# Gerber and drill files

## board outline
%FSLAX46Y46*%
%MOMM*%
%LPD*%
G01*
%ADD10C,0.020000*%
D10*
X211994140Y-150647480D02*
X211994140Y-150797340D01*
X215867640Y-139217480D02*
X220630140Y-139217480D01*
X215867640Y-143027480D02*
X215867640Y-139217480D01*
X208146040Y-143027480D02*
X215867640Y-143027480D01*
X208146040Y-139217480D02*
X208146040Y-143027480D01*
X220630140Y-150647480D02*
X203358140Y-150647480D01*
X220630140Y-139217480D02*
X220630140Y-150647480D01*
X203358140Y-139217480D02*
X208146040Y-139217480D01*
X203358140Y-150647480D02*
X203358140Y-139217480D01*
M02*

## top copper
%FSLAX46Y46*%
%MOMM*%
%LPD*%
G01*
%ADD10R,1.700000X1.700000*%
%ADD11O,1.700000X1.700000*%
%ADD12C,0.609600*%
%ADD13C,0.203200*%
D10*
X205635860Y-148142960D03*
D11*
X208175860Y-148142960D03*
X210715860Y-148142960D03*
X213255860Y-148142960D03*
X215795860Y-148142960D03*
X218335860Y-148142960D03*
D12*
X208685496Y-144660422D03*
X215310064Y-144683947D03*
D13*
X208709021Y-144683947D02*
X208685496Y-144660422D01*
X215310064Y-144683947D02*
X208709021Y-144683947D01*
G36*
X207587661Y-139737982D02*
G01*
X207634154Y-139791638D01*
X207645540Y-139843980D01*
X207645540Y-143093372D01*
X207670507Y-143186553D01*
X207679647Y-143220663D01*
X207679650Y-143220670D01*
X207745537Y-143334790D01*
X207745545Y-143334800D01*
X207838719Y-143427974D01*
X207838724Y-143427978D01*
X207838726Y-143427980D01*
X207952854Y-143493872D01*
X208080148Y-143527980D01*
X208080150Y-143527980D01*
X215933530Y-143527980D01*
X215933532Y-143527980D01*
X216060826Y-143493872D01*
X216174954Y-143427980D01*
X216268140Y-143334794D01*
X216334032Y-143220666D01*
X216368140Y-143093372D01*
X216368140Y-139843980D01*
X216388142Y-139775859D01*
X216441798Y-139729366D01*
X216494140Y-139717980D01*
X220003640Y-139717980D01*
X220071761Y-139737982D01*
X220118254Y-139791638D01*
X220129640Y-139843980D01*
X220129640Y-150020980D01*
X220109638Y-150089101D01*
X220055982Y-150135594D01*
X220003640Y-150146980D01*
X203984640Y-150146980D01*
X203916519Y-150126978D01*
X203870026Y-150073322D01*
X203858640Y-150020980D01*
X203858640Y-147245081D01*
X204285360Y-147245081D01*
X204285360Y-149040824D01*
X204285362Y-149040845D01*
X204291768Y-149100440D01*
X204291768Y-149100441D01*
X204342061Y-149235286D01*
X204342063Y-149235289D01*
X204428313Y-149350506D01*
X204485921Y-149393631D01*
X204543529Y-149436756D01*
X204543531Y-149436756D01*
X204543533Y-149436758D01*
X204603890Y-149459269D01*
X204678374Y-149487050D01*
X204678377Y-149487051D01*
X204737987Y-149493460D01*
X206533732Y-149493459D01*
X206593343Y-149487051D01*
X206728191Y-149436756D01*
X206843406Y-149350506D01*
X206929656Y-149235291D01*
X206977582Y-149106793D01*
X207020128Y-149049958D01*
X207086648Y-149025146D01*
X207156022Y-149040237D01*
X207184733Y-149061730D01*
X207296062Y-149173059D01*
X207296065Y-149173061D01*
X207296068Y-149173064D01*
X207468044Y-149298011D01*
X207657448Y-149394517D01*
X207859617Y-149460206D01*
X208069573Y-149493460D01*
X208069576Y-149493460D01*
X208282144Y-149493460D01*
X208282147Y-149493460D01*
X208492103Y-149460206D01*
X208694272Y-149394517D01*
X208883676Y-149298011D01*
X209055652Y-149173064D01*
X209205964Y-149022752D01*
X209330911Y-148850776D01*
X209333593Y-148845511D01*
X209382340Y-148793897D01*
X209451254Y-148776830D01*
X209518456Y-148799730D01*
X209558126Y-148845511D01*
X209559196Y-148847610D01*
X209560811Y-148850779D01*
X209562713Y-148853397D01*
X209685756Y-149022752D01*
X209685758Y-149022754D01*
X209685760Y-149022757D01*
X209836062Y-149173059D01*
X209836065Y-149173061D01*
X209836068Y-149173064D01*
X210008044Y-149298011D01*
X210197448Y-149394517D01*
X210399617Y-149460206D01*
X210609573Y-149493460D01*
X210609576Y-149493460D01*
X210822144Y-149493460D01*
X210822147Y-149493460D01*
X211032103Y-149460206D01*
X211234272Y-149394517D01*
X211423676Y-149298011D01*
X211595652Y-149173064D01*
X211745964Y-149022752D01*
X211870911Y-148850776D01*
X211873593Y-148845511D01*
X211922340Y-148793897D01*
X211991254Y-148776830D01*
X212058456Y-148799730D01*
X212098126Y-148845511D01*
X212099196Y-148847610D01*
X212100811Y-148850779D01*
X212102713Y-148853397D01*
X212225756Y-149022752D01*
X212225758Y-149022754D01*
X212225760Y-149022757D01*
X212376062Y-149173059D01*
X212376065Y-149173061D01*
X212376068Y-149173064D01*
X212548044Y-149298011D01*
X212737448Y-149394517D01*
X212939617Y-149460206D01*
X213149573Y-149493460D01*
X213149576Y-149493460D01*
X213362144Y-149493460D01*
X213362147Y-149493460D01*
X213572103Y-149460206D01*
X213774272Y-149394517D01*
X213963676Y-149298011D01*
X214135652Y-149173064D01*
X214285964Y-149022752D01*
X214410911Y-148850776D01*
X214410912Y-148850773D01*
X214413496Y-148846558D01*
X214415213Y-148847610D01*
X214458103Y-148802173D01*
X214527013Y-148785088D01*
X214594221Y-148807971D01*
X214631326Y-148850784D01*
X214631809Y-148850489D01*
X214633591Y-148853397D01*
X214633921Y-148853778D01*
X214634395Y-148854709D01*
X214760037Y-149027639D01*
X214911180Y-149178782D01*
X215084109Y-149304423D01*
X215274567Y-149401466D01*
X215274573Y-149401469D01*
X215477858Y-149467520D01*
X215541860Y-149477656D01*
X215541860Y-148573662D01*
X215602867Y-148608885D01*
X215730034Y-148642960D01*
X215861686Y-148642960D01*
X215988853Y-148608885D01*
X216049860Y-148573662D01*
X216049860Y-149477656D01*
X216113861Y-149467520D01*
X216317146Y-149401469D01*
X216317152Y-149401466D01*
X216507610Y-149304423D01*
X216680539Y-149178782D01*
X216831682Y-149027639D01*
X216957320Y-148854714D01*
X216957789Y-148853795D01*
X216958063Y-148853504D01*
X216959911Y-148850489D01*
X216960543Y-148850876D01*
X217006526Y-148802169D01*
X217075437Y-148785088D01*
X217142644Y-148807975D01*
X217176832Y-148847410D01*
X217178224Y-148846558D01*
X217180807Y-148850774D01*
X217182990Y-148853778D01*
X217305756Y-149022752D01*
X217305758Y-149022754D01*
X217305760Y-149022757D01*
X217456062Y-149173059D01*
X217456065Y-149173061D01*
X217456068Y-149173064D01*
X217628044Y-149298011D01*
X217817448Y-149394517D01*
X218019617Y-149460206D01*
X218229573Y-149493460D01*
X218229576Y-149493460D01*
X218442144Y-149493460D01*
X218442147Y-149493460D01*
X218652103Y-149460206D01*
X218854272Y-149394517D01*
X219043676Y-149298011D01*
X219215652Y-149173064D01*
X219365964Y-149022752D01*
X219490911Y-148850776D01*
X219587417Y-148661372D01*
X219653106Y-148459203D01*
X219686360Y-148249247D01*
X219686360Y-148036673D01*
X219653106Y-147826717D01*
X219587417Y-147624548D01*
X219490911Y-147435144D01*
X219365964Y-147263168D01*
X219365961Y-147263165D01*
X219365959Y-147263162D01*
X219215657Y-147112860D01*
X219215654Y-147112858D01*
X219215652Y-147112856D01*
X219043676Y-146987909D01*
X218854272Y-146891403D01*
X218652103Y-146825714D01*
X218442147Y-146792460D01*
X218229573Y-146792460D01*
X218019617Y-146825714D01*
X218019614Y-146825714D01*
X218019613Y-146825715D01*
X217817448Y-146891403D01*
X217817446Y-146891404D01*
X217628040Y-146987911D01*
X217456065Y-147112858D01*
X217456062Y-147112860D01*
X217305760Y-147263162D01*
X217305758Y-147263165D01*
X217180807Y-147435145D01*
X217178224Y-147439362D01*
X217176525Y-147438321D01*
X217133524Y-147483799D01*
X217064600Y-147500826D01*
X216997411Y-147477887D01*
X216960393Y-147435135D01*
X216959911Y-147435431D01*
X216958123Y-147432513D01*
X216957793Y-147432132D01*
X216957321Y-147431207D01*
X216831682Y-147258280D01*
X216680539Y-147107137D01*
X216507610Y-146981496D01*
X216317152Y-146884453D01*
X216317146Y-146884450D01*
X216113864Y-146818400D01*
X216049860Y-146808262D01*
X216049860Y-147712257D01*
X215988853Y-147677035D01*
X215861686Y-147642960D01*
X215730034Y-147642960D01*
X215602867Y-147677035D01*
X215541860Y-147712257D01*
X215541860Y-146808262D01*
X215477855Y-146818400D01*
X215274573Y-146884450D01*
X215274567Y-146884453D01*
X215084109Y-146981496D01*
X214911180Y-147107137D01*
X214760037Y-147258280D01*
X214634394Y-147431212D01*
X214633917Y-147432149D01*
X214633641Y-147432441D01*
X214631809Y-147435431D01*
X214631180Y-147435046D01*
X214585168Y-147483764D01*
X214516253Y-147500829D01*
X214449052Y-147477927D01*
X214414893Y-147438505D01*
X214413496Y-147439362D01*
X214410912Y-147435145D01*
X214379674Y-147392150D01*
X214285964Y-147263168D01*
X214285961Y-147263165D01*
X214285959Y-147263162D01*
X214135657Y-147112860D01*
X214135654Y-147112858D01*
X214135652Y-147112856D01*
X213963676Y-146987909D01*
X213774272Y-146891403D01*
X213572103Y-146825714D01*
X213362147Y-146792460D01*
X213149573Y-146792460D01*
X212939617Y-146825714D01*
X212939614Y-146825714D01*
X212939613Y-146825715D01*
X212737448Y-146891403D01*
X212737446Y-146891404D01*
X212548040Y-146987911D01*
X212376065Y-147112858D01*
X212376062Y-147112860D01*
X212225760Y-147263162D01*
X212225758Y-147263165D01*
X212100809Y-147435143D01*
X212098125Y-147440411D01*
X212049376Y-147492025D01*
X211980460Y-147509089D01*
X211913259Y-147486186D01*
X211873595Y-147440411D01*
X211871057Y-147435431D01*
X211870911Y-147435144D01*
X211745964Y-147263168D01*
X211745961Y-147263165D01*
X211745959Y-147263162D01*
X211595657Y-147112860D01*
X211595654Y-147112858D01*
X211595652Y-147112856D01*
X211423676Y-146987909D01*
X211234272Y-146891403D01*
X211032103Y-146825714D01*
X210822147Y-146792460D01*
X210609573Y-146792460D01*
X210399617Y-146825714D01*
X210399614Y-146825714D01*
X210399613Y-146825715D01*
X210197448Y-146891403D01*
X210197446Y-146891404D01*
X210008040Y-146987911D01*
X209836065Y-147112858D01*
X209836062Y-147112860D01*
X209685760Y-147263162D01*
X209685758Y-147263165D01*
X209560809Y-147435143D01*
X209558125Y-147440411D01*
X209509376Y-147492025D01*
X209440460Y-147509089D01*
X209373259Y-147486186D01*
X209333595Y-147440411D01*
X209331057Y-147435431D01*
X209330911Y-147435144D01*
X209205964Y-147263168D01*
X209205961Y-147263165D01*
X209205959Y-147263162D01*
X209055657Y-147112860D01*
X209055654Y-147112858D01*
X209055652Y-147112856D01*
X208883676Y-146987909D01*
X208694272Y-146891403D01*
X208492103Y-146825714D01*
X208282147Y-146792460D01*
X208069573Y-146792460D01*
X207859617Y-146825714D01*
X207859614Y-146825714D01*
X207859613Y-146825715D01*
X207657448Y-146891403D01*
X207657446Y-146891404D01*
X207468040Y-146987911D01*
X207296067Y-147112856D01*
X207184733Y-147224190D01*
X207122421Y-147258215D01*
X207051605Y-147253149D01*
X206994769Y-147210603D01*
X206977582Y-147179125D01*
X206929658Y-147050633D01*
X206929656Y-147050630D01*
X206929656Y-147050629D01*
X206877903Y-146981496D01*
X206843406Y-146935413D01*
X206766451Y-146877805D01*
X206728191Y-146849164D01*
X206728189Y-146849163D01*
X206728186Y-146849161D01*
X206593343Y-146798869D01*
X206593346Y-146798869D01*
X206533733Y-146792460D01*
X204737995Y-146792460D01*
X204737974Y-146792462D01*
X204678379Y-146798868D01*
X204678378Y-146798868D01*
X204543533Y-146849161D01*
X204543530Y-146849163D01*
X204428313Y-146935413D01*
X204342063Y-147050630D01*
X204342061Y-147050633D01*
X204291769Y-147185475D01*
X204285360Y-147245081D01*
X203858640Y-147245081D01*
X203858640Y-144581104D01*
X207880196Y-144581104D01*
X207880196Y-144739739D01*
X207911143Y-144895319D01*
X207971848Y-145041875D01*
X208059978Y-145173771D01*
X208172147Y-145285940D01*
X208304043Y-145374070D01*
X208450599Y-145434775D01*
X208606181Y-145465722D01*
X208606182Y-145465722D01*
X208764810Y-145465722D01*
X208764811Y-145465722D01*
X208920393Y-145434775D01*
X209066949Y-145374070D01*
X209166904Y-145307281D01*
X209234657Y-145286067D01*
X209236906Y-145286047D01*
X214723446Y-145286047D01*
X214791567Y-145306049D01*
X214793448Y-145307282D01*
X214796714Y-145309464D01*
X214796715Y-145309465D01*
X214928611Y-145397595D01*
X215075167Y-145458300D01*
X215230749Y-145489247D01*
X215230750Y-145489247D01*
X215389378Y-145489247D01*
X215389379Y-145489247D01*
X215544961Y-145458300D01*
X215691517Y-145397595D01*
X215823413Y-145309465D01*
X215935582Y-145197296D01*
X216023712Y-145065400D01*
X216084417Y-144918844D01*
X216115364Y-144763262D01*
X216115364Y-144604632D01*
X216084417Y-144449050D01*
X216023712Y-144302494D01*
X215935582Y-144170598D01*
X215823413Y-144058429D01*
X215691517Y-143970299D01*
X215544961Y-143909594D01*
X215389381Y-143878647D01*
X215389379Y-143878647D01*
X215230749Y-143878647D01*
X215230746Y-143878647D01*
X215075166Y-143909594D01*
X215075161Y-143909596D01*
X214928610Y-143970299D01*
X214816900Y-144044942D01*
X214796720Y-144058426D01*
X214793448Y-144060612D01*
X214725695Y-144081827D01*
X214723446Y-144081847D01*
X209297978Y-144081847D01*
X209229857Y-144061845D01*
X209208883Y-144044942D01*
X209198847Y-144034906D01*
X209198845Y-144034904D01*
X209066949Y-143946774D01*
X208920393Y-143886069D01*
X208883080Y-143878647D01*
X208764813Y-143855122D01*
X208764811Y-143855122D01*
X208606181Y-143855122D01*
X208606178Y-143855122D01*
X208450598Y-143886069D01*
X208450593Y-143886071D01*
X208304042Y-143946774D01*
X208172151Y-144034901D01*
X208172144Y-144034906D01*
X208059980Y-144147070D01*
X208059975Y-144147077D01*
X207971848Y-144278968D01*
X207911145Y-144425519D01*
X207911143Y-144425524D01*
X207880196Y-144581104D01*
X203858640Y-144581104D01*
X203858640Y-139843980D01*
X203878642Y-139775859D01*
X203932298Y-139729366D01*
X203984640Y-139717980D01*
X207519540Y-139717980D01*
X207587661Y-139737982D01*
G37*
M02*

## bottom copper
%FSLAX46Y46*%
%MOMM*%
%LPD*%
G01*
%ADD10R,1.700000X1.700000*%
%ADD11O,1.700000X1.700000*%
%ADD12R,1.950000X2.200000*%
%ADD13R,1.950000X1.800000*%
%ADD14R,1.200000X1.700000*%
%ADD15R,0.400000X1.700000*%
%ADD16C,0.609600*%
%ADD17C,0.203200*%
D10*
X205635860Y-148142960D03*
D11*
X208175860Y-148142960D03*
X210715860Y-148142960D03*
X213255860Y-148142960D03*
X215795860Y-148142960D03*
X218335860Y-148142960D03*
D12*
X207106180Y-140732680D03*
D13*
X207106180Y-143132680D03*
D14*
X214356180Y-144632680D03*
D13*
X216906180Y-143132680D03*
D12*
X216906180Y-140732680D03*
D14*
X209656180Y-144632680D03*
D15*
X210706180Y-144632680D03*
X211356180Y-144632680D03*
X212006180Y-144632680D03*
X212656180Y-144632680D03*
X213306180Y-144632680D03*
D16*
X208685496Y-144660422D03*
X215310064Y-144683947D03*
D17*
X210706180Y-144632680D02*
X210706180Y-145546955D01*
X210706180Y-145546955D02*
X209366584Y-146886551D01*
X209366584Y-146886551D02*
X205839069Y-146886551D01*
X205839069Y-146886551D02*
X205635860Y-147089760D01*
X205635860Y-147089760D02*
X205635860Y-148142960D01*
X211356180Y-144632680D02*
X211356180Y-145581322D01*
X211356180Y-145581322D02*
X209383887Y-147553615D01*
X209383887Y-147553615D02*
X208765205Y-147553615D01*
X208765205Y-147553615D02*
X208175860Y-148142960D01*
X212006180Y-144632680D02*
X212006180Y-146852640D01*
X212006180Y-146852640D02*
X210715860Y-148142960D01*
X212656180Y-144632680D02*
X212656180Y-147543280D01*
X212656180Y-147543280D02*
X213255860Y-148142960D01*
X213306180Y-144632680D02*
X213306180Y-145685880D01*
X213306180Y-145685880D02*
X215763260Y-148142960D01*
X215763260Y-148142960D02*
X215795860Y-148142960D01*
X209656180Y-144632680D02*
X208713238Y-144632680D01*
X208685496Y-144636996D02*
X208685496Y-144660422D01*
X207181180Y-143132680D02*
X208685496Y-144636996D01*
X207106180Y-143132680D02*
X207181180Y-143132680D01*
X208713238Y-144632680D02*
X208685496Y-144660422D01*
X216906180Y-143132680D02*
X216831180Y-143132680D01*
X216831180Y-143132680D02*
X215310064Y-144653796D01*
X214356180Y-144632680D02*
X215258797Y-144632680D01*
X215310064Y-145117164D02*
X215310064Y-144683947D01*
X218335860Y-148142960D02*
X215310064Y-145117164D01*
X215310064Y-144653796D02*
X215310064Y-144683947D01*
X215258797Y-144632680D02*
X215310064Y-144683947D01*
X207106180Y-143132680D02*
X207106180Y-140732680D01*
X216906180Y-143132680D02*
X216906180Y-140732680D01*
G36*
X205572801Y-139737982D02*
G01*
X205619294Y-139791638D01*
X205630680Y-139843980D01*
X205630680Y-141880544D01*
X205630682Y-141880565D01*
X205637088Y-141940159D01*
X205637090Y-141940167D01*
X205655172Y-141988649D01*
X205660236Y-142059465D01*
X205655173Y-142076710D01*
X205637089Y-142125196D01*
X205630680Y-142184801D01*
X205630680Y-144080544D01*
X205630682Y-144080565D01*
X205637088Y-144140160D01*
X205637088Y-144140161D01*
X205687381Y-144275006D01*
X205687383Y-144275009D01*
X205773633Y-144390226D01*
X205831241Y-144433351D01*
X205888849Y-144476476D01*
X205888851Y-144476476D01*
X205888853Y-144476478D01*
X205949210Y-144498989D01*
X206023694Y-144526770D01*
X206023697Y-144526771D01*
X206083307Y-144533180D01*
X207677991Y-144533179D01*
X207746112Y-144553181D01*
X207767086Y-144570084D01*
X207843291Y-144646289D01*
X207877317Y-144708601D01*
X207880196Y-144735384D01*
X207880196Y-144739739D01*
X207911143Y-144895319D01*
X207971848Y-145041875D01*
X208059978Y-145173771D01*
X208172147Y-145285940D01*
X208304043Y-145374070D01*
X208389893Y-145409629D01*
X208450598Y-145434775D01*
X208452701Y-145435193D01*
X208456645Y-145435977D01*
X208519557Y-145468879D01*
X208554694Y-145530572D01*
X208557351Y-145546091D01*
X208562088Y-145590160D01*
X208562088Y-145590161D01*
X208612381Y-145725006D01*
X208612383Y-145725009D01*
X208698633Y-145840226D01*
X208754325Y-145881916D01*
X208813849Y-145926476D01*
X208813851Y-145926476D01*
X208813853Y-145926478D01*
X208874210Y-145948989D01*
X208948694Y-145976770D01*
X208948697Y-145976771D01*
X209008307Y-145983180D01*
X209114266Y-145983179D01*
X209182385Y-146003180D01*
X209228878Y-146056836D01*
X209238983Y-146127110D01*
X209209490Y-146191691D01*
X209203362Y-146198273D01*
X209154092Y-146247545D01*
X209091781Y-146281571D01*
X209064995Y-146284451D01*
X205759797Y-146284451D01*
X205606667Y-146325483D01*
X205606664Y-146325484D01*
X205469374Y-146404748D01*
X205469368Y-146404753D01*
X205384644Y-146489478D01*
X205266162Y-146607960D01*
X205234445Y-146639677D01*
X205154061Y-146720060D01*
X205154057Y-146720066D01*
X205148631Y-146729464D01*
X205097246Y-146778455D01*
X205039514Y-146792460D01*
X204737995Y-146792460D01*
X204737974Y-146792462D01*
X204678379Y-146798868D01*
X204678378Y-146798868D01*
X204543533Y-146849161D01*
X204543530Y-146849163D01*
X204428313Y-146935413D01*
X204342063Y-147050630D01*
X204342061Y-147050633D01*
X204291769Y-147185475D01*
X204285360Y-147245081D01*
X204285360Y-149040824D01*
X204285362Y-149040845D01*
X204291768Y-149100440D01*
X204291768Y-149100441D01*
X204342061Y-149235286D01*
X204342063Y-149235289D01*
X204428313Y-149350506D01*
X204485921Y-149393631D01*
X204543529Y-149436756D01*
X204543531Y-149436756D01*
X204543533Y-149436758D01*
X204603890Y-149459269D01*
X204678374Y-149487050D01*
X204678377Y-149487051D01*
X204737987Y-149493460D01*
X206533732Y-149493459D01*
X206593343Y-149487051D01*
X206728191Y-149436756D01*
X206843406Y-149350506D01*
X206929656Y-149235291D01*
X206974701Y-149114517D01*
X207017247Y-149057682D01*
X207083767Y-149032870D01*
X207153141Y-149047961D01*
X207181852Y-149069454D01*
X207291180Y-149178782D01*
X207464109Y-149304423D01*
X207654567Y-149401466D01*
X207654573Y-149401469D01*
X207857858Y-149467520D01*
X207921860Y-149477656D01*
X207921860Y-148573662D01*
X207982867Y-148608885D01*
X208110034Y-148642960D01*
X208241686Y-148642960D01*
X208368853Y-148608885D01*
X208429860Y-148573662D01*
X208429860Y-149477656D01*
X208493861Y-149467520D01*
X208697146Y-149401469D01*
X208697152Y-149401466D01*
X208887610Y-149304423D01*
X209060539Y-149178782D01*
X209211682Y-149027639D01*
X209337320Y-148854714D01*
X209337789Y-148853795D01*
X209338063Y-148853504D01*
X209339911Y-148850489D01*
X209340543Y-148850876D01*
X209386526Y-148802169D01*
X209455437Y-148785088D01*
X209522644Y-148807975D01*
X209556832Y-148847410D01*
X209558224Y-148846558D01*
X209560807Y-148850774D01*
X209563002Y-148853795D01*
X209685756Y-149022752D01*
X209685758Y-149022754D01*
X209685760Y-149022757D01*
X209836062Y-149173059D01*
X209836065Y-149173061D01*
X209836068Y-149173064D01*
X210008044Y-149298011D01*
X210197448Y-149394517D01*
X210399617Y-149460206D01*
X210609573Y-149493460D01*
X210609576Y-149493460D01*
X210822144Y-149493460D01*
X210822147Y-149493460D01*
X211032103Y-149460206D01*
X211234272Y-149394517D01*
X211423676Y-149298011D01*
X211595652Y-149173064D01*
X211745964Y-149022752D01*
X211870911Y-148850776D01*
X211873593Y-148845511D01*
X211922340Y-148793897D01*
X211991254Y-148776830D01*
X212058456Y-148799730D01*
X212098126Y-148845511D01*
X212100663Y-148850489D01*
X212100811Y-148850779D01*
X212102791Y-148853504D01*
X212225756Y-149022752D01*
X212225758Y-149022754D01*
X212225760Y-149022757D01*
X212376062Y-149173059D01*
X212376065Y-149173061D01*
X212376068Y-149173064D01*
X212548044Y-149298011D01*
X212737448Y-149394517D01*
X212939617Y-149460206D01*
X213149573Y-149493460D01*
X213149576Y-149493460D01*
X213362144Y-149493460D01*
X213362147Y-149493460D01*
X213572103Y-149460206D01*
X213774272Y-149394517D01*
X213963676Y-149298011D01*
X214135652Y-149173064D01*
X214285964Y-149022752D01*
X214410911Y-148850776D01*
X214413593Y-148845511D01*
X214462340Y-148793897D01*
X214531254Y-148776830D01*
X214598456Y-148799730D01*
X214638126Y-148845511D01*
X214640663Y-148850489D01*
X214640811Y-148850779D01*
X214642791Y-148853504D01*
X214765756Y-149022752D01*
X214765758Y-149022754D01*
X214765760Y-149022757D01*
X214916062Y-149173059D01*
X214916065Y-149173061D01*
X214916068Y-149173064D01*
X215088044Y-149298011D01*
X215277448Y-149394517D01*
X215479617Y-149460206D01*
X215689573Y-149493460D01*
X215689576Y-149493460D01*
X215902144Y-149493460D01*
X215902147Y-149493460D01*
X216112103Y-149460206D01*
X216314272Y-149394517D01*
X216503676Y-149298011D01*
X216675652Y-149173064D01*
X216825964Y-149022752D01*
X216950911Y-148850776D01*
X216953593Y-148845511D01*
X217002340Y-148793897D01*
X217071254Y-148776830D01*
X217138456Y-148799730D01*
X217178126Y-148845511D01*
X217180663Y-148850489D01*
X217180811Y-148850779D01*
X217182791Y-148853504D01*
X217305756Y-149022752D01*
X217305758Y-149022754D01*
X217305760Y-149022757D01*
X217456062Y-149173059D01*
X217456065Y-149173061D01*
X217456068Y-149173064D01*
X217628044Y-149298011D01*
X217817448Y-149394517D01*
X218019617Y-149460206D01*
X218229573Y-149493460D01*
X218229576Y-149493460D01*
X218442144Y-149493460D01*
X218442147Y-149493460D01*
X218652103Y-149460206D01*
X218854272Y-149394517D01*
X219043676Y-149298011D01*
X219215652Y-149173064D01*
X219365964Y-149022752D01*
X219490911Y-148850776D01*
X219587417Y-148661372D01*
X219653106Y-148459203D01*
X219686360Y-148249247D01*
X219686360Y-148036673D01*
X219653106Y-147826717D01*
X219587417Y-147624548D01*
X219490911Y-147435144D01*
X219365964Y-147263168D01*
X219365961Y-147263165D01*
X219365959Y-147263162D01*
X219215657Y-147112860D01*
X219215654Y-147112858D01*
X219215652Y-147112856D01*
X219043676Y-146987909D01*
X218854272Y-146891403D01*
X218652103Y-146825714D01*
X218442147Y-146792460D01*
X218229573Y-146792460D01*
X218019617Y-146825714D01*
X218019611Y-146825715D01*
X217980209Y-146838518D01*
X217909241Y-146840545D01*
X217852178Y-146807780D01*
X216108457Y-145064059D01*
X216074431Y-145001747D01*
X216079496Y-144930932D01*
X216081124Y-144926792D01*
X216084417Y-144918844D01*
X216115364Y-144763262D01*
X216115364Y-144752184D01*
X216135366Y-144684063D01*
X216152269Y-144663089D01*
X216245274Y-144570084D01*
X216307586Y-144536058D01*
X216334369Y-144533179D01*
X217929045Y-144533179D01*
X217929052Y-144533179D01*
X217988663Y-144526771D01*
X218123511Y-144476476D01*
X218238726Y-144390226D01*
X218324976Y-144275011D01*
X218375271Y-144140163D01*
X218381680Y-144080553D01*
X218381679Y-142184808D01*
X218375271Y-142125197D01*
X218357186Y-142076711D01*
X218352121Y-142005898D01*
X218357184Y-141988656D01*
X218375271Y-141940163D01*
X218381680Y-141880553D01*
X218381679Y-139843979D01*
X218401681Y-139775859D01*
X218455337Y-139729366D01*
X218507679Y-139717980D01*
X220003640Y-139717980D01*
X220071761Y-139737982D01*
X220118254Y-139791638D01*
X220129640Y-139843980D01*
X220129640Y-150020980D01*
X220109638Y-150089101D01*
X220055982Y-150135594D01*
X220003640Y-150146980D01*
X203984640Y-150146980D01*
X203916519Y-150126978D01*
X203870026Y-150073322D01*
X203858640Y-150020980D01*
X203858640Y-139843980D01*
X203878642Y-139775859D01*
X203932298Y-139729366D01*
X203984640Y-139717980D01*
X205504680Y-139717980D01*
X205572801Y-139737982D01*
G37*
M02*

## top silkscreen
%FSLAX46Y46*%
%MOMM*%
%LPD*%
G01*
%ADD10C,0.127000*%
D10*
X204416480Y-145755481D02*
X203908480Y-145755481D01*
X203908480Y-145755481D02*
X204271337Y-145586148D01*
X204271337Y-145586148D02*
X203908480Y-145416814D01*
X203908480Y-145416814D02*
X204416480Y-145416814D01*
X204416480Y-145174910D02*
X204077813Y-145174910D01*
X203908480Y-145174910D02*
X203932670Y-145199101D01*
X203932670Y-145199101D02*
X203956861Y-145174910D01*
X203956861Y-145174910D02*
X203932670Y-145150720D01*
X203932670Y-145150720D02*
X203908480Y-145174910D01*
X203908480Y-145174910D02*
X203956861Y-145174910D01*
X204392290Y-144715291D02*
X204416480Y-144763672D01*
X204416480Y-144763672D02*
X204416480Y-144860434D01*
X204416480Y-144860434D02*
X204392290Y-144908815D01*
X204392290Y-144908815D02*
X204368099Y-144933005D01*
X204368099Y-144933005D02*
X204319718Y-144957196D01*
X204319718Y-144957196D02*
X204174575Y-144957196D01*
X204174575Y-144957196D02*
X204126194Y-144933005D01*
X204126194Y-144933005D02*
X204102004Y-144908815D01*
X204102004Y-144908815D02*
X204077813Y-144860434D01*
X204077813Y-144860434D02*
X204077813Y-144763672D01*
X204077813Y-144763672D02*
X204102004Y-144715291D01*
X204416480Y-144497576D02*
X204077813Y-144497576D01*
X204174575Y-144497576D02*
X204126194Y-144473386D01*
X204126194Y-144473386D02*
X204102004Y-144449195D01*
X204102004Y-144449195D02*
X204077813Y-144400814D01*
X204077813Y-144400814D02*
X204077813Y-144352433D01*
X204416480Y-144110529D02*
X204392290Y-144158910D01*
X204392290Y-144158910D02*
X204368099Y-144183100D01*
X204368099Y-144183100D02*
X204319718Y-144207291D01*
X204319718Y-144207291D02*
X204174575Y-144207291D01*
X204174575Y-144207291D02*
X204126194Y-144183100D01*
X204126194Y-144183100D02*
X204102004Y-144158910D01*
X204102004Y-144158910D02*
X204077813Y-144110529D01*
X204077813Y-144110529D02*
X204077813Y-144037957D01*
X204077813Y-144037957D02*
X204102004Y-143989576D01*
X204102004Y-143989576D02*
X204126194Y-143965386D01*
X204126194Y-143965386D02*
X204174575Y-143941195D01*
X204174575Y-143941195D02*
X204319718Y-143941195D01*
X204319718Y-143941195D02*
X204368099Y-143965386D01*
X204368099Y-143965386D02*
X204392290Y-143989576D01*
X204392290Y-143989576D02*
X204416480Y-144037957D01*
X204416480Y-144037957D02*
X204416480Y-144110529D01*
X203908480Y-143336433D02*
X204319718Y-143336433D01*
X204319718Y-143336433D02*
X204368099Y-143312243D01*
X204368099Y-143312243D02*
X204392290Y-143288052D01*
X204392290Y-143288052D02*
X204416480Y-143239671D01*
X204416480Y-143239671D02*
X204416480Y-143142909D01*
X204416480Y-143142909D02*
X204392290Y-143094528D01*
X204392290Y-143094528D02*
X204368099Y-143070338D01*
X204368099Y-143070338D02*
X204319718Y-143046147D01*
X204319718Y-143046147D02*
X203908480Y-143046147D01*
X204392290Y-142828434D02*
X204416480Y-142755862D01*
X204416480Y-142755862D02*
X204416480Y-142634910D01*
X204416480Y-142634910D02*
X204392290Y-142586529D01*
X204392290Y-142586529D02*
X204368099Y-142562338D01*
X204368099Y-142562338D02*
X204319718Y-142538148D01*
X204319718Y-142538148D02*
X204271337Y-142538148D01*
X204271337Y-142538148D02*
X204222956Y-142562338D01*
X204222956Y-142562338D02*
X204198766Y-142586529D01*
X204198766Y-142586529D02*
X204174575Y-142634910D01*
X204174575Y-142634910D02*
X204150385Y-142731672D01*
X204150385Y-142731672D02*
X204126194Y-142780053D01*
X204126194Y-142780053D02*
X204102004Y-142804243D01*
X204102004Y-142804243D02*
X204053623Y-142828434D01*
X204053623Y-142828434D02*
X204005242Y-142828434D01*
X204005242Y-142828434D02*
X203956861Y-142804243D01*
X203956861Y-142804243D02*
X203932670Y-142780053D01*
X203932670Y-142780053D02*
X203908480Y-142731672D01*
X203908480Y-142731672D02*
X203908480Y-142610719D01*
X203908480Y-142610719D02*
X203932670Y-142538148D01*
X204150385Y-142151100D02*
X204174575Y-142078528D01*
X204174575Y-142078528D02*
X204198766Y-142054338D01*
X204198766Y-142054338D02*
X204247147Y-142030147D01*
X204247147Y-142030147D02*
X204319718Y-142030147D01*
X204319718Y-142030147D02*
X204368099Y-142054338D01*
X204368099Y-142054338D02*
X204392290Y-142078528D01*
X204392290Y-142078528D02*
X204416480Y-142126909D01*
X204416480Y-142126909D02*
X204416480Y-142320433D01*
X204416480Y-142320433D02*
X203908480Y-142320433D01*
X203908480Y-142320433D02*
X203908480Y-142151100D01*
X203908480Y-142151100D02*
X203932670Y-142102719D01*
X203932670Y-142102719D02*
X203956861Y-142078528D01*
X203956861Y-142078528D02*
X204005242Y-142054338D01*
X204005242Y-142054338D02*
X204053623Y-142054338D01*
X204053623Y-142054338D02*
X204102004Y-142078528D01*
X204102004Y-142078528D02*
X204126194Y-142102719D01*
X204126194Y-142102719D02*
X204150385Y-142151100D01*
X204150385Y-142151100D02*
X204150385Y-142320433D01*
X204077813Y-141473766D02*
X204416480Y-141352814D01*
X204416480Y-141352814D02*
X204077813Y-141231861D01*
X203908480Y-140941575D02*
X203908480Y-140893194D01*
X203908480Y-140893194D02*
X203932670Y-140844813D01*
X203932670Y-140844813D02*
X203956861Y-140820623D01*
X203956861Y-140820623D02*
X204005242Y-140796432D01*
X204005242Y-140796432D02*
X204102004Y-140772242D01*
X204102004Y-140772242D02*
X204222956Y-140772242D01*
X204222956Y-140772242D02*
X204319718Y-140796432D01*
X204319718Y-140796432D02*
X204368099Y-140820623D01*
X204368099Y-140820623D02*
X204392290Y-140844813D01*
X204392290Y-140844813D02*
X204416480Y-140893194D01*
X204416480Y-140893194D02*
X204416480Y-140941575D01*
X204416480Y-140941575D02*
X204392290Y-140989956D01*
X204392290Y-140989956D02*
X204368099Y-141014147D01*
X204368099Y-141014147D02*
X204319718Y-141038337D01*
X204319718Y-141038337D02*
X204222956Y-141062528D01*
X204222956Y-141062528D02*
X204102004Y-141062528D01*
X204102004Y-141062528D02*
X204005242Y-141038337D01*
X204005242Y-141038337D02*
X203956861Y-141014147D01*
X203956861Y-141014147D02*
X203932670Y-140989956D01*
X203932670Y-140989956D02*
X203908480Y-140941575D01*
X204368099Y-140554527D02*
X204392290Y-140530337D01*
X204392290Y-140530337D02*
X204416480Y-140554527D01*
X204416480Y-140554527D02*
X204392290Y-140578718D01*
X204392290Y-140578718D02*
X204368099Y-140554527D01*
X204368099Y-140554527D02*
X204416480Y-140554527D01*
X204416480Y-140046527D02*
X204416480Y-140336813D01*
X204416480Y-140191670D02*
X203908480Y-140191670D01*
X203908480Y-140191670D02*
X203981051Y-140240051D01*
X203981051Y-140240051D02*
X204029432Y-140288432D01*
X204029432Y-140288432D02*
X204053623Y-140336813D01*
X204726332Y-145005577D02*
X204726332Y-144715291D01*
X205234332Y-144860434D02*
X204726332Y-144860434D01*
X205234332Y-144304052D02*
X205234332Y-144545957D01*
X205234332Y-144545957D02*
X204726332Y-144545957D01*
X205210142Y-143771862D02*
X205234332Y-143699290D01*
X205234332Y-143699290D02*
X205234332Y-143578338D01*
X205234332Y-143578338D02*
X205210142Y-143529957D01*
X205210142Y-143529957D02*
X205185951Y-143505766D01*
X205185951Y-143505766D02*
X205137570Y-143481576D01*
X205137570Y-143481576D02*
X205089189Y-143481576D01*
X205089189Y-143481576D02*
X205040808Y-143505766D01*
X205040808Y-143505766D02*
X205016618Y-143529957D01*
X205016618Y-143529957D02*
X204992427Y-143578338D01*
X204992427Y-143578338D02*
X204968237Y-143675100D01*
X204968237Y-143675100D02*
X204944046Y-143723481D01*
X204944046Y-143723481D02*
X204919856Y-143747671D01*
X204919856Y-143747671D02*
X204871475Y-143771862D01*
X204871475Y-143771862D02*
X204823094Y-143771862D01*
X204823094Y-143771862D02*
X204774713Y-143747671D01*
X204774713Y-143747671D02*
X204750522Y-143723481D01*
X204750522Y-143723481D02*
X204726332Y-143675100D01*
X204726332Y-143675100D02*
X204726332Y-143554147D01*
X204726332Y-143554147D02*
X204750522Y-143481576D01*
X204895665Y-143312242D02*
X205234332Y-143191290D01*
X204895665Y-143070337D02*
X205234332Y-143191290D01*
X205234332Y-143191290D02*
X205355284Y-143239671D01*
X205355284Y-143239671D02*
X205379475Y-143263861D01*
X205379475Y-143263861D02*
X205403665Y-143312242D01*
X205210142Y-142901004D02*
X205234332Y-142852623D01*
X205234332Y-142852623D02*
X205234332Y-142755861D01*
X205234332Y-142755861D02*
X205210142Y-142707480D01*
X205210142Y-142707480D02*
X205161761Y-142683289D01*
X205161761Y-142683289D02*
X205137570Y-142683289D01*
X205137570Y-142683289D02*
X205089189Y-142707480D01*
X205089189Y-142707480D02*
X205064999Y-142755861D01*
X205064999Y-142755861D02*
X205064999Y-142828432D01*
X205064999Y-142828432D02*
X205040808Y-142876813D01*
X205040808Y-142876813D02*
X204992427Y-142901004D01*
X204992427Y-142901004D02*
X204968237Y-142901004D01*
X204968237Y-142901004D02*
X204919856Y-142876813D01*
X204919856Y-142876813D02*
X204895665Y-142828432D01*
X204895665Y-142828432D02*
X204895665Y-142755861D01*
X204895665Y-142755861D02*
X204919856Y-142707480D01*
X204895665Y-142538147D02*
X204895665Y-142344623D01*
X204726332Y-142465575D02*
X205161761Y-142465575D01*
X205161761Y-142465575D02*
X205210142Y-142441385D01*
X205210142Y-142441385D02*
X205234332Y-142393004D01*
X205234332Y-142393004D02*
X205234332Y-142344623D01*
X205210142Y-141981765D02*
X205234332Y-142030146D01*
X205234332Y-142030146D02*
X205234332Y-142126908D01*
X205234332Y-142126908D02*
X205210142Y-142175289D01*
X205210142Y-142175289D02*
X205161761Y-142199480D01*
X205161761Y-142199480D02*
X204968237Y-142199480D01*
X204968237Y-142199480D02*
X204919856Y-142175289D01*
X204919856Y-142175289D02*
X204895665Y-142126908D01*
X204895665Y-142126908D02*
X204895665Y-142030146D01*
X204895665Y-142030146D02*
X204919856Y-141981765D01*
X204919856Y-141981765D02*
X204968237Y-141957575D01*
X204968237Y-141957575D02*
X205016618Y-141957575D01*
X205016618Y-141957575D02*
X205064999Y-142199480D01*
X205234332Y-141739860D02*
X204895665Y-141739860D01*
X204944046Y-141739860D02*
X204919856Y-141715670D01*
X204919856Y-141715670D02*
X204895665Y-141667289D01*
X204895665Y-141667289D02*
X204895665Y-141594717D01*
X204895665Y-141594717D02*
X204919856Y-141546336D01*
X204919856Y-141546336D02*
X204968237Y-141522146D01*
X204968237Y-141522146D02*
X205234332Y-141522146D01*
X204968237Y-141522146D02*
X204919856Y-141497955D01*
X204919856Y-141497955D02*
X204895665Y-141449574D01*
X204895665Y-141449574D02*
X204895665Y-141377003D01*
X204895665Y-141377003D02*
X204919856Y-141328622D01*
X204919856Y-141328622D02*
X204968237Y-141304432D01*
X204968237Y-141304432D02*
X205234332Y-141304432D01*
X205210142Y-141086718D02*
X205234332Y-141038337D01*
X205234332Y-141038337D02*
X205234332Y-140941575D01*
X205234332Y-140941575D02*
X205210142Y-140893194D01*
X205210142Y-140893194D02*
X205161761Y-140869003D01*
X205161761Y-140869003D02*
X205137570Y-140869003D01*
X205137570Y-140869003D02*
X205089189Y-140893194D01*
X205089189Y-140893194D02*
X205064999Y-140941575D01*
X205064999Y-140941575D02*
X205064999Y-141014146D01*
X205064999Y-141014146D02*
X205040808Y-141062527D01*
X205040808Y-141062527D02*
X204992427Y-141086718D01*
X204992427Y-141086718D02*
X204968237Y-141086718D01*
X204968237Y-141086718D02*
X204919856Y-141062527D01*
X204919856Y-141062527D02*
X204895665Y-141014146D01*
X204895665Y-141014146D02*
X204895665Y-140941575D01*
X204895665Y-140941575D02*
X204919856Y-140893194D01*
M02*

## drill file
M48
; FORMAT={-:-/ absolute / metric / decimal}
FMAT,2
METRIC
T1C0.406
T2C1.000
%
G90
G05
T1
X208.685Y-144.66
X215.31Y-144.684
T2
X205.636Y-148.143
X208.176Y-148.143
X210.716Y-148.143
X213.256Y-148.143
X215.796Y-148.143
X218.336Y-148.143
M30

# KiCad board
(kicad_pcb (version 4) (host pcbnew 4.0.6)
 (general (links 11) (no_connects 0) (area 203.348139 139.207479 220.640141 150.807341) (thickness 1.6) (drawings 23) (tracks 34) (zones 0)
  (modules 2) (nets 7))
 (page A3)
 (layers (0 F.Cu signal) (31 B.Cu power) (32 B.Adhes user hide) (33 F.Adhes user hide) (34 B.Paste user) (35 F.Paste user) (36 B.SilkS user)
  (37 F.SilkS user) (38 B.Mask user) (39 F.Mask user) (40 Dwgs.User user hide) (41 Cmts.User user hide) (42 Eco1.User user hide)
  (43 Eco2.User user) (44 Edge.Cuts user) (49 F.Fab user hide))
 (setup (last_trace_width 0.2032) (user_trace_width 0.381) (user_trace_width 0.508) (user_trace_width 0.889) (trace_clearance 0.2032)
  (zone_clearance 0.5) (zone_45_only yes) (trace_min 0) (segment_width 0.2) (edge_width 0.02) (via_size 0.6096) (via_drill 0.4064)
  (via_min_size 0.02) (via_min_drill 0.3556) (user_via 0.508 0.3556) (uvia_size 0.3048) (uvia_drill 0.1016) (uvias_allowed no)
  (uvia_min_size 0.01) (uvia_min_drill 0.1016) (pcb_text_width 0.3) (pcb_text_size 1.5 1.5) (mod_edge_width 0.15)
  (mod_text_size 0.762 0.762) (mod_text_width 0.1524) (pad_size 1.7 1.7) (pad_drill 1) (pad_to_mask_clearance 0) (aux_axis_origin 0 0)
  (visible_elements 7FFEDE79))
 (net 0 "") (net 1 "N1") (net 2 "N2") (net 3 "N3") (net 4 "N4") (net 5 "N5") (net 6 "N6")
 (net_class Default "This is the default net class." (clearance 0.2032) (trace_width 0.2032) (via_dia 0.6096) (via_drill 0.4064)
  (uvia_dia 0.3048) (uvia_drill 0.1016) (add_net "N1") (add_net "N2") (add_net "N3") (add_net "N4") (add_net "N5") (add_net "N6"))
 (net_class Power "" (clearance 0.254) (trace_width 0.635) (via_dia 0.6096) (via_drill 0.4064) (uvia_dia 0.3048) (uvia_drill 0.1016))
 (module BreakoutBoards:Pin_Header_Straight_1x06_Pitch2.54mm (layer B.Cu) (at 205.63586 148.14296 270)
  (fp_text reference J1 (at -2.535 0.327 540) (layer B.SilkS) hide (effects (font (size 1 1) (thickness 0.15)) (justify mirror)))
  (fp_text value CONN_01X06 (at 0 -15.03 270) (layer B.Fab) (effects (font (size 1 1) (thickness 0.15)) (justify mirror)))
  (pad 1 thru_hole rect (at 0 0 270) (size 1.7 1.7) (drill 1) (layers *.Cu *.Mask) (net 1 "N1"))
  (pad 2 thru_hole oval (at 0 -2.54 270) (size 1.7 1.7) (drill 1) (layers *.Cu *.Mask) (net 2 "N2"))
  (pad 3 thru_hole oval (at 0 -5.08 270) (size 1.7 1.7) (drill 1) (layers *.Cu *.Mask) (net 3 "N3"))
  (pad 4 thru_hole oval (at 0 -7.62 270) (size 1.7 1.7) (drill 1) (layers *.Cu *.Mask) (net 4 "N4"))
  (pad 5 thru_hole oval (at 0 -10.16 270) (size 1.7 1.7) (drill 1) (layers *.Cu *.Mask) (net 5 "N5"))
  (pad 6 thru_hole oval (at 0 -12.7 270) (size 1.7 1.7) (drill 1) (layers *.Cu *.Mask) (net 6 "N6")))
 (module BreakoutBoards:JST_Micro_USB (layer B.Cu) (at 212.00618 140.73268)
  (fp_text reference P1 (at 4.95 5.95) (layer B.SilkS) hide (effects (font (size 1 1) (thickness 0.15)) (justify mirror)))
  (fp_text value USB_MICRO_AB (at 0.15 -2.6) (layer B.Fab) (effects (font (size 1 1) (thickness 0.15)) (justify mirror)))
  (pad 6 smd rect (at -4.9 0 180) (size 1.95 2.2) (layers B.Cu B.Paste B.Mask) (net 6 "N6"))
  (pad 6 smd rect (at -4.9 2.4) (size 1.95 1.8) (layers B.Cu B.Paste B.Mask) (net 6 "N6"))
  (pad 6 smd rect (at 2.35 3.9) (size 1.2 1.7) (layers B.Cu B.Paste B.Mask) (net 6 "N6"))
  (pad 6 smd rect (at 4.9 2.4 180) (size 1.95 1.8) (layers B.Cu B.Paste B.Mask) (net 6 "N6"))
  (pad 6 smd rect (at 4.9 0 180) (size 1.95 2.2) (layers B.Cu B.Paste B.Mask) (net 6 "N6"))
  (pad 6 smd rect (at -2.35 3.9) (size 1.2 1.7) (layers B.Cu B.Paste B.Mask) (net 6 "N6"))
  (pad 1 smd rect (at -1.3 3.9) (size 0.4 1.7) (layers B.Cu B.Paste B.Mask) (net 1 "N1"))
  (pad 2 smd rect (at -0.65 3.9) (size 0.4 1.7) (layers B.Cu B.Paste B.Mask) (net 2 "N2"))
  (pad 3 smd rect (at 0 3.9) (size 0.4 1.7) (layers B.Cu B.Paste B.Mask) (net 3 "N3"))
  (pad 4 smd rect (at 0.65 3.9) (size 0.4 1.7) (layers B.Cu B.Paste B.Mask) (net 4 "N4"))
  (pad 5 smd rect (at 1.3 3.9) (size 0.4 1.7) (layers B.Cu B.Paste B.Mask) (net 5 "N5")))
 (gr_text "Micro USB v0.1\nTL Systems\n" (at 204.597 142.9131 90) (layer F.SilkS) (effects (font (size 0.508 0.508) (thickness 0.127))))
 (gr_line (start 211.99414 150.64748) (end 211.99414 150.79734) (layer Edge.Cuts) (width 0.02))
 (gr_line (start 215.86764 139.21748) (end 220.63014 139.21748) (layer Edge.Cuts) (width 0.02))
 (gr_line (start 215.86764 143.02748) (end 215.86764 139.21748) (layer Edge.Cuts) (width 0.02))
 (gr_line (start 208.14604 143.02748) (end 215.86764 143.02748) (layer Edge.Cuts) (width 0.02))
 (gr_line (start 208.14604 139.21748) (end 208.14604 143.02748) (layer Edge.Cuts) (width 0.02))
 (gr_line (start 220.63014 150.64748) (end 203.35814 150.64748) (layer Edge.Cuts) (width 0.02))
 (gr_line (start 220.63014 139.21748) (end 220.63014 150.64748) (layer Edge.Cuts) (width 0.02))
 (gr_line (start 203.35814 139.21748) (end 208.14604 139.21748) (layer Edge.Cuts) (width 0.02))
 (gr_line (start 203.35814 150.64748) (end 203.35814 139.21748) (layer Edge.Cuts) (width 0.02))
 (segment (start 210.70618 144.63268) (end 210.70618 145.546955) (width 0.2032) (layer B.Cu) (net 1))
 (segment (start 210.70618 145.546955) (end 209.366584 146.886551) (width 0.2032) (layer B.Cu) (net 1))
 (segment (start 209.366584 146.886551) (end 205.839069 146.886551) (width 0.2032) (layer B.Cu) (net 1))
 (segment (start 205.839069 146.886551) (end 205.63586 147.08976) (width 0.2032) (layer B.Cu) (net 1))
 (segment (start 205.63586 147.08976) (end 205.63586 148.14296) (width 0.2032) (layer B.Cu) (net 1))
 (segment (start 211.35618 144.63268) (end 211.35618 145.581322) (width 0.2032) (layer B.Cu) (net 2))
 (segment (start 211.35618 145.581322) (end 209.383887 147.553615) (width 0.2032) (layer B.Cu) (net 2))
 (segment (start 209.383887 147.553615) (end 208.765205 147.553615) (width 0.2032) (layer B.Cu) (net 2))
 (segment (start 208.765205 147.553615) (end 208.17586 148.14296) (width 0.2032) (layer B.Cu) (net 2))
 (segment (start 212.00618 144.63268) (end 212.00618 146.85264) (width 0.2032) (layer B.Cu) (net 3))
 (segment (start 212.00618 146.85264) (end 210.71586 148.14296) (width 0.2032) (layer B.Cu) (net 3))
 (segment (start 212.65618 144.63268) (end 212.65618 147.54328) (width 0.2032) (layer B.Cu) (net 4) (status 30))
 (segment (start 212.65618 147.54328) (end 213.25586 148.14296) (width 0.2032) (layer B.Cu) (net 4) (status 30))
 (segment (start 213.30618 144.63268) (end 213.30618 145.68588) (width 0.2032) (layer B.Cu) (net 5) (status 10))
 (segment (start 213.30618 145.68588) (end 215.76326 148.14296) (width 0.2032) (layer B.Cu) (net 5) (status 20))
 (segment (start 215.76326 148.14296) (end 215.79586 148.14296) (width 0.2032) (layer B.Cu) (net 5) (status 30))
 (segment (start 209.65618 144.63268) (end 208.713238 144.63268) (width 0.2032) (layer B.Cu) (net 6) (status 10))
 (segment (start 208.685496 144.636996) (end 208.685496 144.660422) (width 0.2032) (layer B.Cu) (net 6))
 (segment (start 207.18118 143.13268) (end 208.685496 144.636996) (width 0.2032) (layer B.Cu) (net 6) (status 10))
 (segment (start 207.10618 143.13268) (end 207.18118 143.13268) (width 0.2032) (layer B.Cu) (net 6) (status 30))
 (segment (start 208.709021 144.683947) (end 208.685496 144.660422) (width 0.2032) (layer F.Cu) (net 6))
 (segment (start 208.713238 144.63268) (end 208.685496 144.660422) (width 0.2032) (layer B.Cu) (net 6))
 (segment (start 215.310064 144.683947) (end 208.709021 144.683947) (width 0.2032) (layer F.Cu) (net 6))
 (via (at 208.685496 144.660422) (size 0.6096) (drill 0.4064) (layers F.Cu B.Cu) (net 6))
 (segment (start 216.90618 143.13268) (end 216.83118 143.13268) (width 0.2032) (layer B.Cu) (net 6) (status 30))
 (segment (start 216.83118 143.13268) (end 215.310064 144.653796) (width 0.2032) (layer B.Cu) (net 6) (status 10))
 (segment (start 214.35618 144.63268) (end 215.258797 144.63268) (width 0.2032) (layer B.Cu) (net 6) (status 10))
 (segment (start 215.310064 145.117164) (end 215.310064 144.683947) (width 0.2032) (layer B.Cu) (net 6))
 (segment (start 218.33586 148.14296) (end 215.310064 145.117164) (width 0.2032) (layer B.Cu) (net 6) (status 10))
 (segment (start 215.310064 144.653796) (end 215.310064 144.683947) (width 0.2032) (layer B.Cu) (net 6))
 (segment (start 215.258797 144.63268) (end 215.310064 144.683947) (width 0.2032) (layer B.Cu) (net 6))
 (via (at 215.310064 144.683947) (size 0.6096) (drill 0.4064) (layers F.Cu B.Cu) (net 6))
 (segment (start 207.10618 143.13268) (end 207.10618 140.73268) (width 0.2032) (layer B.Cu) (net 6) (status 30))
 (segment (start 216.90618 143.13268) (end 216.90618 140.73268) (width 0.2032) (layer B.Cu) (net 6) (status 30))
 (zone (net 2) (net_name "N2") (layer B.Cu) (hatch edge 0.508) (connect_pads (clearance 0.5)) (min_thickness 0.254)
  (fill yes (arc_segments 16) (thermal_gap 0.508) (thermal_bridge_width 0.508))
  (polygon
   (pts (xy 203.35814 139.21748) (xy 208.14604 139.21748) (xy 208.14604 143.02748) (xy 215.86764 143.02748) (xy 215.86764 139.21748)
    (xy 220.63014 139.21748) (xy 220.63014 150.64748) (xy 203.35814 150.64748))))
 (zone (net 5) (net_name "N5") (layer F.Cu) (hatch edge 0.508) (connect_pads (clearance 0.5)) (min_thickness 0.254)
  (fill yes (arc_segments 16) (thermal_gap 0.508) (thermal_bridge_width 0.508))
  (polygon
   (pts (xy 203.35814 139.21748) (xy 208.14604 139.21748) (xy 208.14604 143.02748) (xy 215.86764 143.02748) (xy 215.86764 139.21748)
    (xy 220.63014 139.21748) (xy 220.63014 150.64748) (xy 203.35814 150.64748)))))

